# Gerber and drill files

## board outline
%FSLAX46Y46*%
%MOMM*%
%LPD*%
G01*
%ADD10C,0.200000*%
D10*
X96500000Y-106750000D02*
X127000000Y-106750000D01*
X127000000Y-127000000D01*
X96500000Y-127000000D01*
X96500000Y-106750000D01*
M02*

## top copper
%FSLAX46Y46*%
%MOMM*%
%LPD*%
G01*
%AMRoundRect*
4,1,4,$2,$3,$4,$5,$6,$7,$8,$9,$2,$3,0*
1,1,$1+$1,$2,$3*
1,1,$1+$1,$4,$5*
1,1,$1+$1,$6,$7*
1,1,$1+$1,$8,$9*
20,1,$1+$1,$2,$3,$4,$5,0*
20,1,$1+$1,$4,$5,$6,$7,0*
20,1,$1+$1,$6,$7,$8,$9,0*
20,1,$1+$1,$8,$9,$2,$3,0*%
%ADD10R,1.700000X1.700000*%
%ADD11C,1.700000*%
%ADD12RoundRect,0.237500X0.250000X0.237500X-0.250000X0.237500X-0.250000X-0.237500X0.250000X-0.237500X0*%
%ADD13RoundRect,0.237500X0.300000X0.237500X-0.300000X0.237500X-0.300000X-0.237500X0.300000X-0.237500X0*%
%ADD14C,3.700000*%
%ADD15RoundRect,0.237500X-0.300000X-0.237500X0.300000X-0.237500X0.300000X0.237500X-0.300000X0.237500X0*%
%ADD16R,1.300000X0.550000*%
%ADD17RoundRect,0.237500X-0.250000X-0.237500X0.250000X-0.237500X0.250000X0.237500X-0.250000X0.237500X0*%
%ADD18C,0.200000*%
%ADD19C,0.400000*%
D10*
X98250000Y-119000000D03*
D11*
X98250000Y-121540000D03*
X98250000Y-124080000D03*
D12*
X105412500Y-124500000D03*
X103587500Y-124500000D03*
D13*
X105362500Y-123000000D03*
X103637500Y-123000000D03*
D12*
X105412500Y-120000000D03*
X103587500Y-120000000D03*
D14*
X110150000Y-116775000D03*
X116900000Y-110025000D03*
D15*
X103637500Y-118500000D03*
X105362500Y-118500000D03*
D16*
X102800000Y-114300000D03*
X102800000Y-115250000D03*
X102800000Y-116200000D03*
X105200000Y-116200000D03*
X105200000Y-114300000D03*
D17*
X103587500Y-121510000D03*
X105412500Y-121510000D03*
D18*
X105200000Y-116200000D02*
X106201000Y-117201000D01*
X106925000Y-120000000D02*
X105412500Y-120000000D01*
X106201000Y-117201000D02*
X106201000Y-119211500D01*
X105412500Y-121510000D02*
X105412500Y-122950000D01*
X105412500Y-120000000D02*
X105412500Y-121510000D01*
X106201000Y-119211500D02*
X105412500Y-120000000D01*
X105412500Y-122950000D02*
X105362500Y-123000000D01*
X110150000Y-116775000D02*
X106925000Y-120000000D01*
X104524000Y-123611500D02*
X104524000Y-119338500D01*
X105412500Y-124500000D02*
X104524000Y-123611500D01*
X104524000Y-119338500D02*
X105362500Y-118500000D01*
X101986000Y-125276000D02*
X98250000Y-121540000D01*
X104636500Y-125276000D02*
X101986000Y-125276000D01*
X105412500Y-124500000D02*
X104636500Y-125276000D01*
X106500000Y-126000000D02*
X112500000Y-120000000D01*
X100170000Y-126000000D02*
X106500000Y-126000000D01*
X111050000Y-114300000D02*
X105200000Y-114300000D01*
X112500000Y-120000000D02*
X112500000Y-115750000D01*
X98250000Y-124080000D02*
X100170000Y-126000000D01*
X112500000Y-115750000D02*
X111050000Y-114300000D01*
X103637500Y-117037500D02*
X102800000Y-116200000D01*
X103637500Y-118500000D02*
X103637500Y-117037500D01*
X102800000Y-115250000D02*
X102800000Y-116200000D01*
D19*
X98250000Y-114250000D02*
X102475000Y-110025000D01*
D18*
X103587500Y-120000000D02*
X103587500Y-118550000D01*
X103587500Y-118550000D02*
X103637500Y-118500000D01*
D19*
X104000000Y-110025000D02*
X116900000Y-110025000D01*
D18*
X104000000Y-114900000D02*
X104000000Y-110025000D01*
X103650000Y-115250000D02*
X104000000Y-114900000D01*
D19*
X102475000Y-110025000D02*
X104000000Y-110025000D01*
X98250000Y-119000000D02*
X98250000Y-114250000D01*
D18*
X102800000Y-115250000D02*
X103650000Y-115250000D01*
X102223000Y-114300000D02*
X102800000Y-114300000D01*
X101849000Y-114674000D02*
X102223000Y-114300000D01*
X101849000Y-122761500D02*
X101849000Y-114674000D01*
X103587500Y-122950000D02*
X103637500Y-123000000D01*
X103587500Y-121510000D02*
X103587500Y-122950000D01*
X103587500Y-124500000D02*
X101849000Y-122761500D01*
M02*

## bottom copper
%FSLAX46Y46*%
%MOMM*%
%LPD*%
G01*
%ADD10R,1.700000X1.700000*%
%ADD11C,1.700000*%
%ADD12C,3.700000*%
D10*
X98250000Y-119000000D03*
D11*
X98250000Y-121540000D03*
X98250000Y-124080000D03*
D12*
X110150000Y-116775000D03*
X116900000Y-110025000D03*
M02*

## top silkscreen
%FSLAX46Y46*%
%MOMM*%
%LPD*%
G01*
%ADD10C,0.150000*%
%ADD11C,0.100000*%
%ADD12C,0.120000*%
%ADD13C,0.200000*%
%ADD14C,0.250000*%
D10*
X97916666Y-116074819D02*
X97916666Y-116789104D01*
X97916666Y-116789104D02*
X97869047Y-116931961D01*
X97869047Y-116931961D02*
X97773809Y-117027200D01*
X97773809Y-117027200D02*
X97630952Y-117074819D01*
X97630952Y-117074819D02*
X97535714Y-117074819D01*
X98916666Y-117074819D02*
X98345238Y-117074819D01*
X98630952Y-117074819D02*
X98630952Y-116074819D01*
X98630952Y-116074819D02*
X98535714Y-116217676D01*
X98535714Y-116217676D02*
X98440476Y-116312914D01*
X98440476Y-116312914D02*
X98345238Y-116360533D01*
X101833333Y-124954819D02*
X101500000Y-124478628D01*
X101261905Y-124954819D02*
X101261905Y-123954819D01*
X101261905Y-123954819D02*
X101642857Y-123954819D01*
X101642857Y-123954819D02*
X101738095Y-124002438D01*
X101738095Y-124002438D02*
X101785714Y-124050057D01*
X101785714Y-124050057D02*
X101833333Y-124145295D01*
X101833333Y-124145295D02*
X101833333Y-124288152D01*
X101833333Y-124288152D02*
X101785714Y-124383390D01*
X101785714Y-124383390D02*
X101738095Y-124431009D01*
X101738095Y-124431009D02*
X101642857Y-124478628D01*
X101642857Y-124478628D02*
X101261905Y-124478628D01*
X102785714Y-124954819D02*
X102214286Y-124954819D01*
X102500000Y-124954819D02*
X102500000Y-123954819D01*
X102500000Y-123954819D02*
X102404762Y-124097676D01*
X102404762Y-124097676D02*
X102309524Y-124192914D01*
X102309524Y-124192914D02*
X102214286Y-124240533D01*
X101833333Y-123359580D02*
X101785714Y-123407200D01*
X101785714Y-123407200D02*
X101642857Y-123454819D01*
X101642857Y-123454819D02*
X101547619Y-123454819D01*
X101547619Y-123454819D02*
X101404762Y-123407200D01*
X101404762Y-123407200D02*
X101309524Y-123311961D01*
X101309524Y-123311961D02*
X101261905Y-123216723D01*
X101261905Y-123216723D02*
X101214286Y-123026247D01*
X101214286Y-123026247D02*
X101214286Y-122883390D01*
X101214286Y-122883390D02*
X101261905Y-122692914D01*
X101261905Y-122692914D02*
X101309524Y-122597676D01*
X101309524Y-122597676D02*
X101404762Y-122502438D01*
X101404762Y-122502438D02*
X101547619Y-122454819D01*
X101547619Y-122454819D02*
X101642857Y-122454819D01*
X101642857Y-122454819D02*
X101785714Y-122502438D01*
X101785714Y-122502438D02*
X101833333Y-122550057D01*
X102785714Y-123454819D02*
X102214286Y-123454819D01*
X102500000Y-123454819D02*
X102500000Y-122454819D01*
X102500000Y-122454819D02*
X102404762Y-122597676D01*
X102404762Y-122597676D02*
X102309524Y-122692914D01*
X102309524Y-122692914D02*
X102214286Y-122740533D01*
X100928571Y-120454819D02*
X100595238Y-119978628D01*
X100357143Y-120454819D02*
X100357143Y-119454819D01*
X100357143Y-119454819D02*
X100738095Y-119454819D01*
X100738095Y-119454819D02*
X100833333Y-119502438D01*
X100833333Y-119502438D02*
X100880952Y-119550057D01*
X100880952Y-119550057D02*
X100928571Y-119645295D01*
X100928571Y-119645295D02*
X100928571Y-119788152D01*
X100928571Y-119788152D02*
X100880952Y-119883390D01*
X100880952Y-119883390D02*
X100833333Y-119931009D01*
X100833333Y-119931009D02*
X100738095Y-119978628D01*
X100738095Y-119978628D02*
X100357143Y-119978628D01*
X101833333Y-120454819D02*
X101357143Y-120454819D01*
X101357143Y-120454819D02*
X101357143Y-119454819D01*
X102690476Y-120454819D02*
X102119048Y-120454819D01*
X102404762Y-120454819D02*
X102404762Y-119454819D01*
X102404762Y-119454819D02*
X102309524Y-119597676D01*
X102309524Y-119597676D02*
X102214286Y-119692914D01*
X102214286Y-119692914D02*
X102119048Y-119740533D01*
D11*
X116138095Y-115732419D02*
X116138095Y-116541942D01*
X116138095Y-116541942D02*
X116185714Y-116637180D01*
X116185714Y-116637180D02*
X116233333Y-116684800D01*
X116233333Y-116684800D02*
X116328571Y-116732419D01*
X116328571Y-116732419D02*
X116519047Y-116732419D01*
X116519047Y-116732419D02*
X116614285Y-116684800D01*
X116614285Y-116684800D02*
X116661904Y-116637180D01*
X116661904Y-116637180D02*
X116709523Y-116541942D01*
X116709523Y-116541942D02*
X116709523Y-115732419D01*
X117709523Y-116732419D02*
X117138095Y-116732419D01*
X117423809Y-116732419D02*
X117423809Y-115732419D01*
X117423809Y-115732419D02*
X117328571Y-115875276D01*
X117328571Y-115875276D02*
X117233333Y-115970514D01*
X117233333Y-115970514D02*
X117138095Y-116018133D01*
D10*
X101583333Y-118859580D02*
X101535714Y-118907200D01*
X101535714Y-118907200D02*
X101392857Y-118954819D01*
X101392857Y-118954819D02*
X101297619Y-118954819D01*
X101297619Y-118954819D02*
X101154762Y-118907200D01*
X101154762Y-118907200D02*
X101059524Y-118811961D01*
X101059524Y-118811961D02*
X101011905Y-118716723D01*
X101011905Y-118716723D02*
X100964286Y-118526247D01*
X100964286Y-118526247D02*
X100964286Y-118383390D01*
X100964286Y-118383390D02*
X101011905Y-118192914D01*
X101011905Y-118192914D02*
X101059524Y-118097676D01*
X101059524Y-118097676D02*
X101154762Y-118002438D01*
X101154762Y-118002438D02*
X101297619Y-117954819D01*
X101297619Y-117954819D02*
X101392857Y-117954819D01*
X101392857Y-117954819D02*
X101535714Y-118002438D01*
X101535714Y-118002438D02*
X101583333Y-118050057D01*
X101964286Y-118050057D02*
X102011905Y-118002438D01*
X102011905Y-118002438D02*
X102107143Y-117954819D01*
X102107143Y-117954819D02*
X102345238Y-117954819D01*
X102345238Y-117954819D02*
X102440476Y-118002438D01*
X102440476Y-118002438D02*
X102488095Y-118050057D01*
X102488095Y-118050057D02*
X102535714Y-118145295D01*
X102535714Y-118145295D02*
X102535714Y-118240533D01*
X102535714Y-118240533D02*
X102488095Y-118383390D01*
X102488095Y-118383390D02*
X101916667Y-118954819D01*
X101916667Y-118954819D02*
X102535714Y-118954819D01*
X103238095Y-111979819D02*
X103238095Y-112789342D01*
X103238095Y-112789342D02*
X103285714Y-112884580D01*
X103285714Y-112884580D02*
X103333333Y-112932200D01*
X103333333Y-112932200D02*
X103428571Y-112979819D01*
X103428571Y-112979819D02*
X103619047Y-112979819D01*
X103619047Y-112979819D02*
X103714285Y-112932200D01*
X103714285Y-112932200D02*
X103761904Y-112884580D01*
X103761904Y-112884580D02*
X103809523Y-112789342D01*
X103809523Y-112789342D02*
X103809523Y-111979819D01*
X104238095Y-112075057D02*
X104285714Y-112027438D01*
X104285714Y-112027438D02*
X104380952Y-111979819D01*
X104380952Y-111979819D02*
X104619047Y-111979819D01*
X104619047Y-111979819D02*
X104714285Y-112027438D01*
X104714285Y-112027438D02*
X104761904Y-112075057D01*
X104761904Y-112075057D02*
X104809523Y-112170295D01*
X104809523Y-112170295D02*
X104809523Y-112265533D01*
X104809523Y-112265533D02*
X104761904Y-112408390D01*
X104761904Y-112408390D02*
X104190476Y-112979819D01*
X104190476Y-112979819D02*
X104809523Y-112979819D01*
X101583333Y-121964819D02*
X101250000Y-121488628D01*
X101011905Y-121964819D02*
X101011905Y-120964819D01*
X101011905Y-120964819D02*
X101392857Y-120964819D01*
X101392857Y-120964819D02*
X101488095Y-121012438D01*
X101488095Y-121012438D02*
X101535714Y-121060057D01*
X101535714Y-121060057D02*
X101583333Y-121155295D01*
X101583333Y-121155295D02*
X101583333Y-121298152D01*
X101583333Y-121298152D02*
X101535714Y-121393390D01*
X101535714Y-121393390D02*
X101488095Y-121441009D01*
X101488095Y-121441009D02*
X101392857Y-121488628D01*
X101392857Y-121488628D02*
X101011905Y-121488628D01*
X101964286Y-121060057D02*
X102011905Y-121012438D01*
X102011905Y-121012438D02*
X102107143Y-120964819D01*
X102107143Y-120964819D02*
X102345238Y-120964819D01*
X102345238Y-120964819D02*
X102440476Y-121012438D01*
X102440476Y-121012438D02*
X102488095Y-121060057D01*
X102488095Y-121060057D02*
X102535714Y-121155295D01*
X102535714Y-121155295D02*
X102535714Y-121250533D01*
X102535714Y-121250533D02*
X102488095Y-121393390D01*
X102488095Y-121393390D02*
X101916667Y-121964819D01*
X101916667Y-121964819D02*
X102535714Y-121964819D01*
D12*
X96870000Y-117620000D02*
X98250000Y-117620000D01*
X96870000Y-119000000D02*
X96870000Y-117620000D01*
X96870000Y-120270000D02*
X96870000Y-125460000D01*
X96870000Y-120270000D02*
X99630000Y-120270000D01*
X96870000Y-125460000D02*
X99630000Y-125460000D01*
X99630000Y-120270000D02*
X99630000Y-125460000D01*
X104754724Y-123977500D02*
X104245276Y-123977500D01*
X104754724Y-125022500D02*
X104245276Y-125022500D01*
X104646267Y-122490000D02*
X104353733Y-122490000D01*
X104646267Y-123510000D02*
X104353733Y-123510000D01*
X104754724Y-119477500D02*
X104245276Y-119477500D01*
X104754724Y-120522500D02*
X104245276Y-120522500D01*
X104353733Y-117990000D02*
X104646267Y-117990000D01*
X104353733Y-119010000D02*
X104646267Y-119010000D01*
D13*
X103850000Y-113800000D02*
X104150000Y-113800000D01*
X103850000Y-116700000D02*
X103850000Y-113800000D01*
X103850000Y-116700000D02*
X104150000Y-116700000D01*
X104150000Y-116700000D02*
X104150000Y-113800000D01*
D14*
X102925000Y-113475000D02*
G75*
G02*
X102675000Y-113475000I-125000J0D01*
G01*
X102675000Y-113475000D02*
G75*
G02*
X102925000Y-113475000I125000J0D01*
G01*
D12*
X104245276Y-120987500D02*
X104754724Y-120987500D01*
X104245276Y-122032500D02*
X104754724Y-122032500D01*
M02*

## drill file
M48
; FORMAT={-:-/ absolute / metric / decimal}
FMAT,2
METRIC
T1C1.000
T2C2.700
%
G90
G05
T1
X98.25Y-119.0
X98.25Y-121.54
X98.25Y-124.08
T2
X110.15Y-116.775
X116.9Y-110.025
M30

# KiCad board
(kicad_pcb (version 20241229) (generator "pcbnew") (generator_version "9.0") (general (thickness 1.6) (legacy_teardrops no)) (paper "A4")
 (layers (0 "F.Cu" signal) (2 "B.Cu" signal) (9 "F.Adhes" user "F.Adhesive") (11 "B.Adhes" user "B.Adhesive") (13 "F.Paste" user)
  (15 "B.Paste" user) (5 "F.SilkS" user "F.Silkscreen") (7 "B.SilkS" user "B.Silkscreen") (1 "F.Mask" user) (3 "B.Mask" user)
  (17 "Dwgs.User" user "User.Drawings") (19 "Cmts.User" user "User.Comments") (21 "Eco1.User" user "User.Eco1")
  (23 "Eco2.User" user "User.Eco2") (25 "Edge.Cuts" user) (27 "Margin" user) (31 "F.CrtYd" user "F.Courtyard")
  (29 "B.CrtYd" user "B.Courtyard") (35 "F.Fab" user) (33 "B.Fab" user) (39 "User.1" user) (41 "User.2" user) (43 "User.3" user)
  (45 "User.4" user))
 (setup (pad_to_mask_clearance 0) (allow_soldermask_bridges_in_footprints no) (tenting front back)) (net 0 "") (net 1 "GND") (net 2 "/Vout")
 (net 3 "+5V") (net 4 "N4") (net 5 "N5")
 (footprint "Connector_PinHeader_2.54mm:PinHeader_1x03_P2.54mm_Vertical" (layer "F.Cu") (at 98.25 119)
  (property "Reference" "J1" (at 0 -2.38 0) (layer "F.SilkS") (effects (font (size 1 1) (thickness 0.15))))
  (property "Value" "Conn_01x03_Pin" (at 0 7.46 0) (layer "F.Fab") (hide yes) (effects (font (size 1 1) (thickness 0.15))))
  (fp_line (start -1.38 -1.38) (end 0 -1.38) (stroke (width 0.12) (type solid)) (layer "F.SilkS"))
  (fp_line (start -1.38 0) (end -1.38 -1.38) (stroke (width 0.12) (type solid)) (layer "F.SilkS"))
  (fp_line (start -1.38 1.27) (end -1.38 6.46) (stroke (width 0.12) (type solid)) (layer "F.SilkS"))
  (fp_line (start -1.38 1.27) (end 1.38 1.27) (stroke (width 0.12) (type solid)) (layer "F.SilkS"))
  (fp_line (start -1.38 6.46) (end 1.38 6.46) (stroke (width 0.12) (type solid)) (layer "F.SilkS"))
  (fp_line (start 1.38 1.27) (end 1.38 6.46) (stroke (width 0.12) (type solid)) (layer "F.SilkS"))
  (pad "1" thru_hole rect (at 0 0) (size 1.7 1.7) (drill 1) (layers "*.Cu" "*.Mask") (remove_unused_layers no) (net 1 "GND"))
  (pad "2" thru_hole circle (at 0 2.54) (size 1.7 1.7) (drill 1) (layers "*.Cu" "*.Mask") (remove_unused_layers no) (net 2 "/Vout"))
  (pad "3" thru_hole circle (at 0 5.08) (size 1.7 1.7) (drill 1) (layers "*.Cu" "*.Mask") (remove_unused_layers no) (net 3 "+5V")))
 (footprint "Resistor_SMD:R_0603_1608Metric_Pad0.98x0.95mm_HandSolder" (layer "F.Cu") (at 104.5 124.5 180)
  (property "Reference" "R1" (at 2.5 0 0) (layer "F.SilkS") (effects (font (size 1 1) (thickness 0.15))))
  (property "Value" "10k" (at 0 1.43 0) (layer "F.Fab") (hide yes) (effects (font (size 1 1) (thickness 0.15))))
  (fp_line (start -0.254724 0.5225) (end 0.254724 0.5225) (stroke (width 0.12) (type solid)) (layer "F.SilkS"))
  (fp_line (start -0.254724 -0.5225) (end 0.254724 -0.5225) (stroke (width 0.12) (type solid)) (layer "F.SilkS"))
  (pad "1" smd roundrect (at -0.9125 0 180) (size 0.975 0.95) (layers "F.Cu" "F.Mask" "F.Paste") (roundrect_rratio 0.25) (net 2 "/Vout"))
  (pad "2" smd roundrect (at 0.9125 0 180) (size 0.975 0.95) (layers "F.Cu" "F.Mask" "F.Paste") (roundrect_rratio 0.25) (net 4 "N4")))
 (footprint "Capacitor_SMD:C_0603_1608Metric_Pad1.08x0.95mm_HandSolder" (layer "F.Cu") (at 104.5 123 180)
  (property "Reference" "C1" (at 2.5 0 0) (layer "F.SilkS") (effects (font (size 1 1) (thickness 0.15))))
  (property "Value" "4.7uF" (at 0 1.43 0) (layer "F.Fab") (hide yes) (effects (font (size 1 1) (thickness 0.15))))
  (fp_line (start -0.146267 0.51) (end 0.146267 0.51) (stroke (width 0.12) (type solid)) (layer "F.SilkS"))
  (fp_line (start -0.146267 -0.51) (end 0.146267 -0.51) (stroke (width 0.12) (type solid)) (layer "F.SilkS"))
  (pad "1" smd roundrect (at -0.8625 0 180) (size 1.075 0.95) (layers "F.Cu" "F.Mask" "F.Paste") (roundrect_rratio 0.25) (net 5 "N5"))
  (pad "2" smd roundrect (at 0.8625 0 180) (size 1.075 0.95) (layers "F.Cu" "F.Mask" "F.Paste") (roundrect_rratio 0.25) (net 4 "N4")))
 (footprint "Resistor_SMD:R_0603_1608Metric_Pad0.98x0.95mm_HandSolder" (layer "F.Cu") (at 104.5 120 180)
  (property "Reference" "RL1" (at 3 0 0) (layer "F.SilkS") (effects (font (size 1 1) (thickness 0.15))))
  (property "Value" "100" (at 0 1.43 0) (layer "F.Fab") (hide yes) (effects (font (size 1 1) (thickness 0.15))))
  (fp_line (start -0.254724 0.5225) (end 0.254724 0.5225) (stroke (width 0.12) (type solid)) (layer "F.SilkS"))
  (fp_line (start -0.254724 -0.5225) (end 0.254724 -0.5225) (stroke (width 0.12) (type solid)) (layer "F.SilkS"))
  (pad "1" smd roundrect (at -0.9125 0 180) (size 0.975 0.95) (layers "F.Cu" "F.Mask" "F.Paste") (roundrect_rratio 0.25) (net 5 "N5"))
  (pad "2" smd roundrect (at 0.9125 0 180) (size 0.975 0.95) (layers "F.Cu" "F.Mask" "F.Paste") (roundrect_rratio 0.25) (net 1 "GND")))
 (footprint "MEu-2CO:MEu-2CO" (layer "F.Cu") (at 116.9 116.775)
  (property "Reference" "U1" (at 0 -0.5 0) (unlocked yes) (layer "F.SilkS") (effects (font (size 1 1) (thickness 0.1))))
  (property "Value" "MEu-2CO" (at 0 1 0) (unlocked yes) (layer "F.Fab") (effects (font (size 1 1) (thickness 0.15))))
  (pad "1" thru_hole circle (at -6.75 0) (size 3.7 3.7) (drill 2.7) (layers "*.Cu" "*.Mask") (remove_unused_layers no) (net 5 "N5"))
  (pad "2" thru_hole circle (at 0 -6.75) (size 3.7 3.7) (drill 2.7) (layers "*.Cu" "*.Mask") (remove_unused_layers no) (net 1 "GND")))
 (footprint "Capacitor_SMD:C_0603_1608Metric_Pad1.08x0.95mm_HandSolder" (layer "F.Cu") (at 104.5 118.5)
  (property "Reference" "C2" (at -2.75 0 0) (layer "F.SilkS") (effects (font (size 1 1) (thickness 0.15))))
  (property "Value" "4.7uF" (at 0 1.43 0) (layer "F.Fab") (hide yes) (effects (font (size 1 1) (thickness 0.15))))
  (fp_line (start -0.146267 -0.51) (end 0.146267 -0.51) (stroke (width 0.12) (type solid)) (layer "F.SilkS"))
  (fp_line (start -0.146267 0.51) (end 0.146267 0.51) (stroke (width 0.12) (type solid)) (layer "F.SilkS"))
  (pad "1" smd roundrect (at -0.8625 0) (size 1.075 0.95) (layers "F.Cu" "F.Mask" "F.Paste") (roundrect_rratio 0.25) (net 1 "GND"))
  (pad "2" smd roundrect (at 0.8625 0) (size 1.075 0.95) (layers "F.Cu" "F.Mask" "F.Paste") (roundrect_rratio 0.25) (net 2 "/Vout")))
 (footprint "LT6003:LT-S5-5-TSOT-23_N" (layer "F.Cu") (at 104 115.25)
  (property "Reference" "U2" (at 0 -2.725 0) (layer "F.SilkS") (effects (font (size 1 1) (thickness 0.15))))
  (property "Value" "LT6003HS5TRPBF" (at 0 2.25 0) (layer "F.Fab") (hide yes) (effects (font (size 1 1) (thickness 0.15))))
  (fp_line (start -0.15 -1.45) (end 0.15 -1.45) (stroke (width 0.2) (type solid)) (layer "F.SilkS"))
  (fp_line (start -0.15 1.45) (end -0.15 -1.45) (stroke (width 0.2) (type solid)) (layer "F.SilkS"))
  (fp_line (start -0.15 1.45) (end 0.15 1.45) (stroke (width 0.2) (type solid)) (layer "F.SilkS"))
  (fp_line (start 0.15 1.45) (end 0.15 -1.45) (stroke (width 0.2) (type solid)) (layer "F.SilkS"))
  (fp_circle (center -1.2 -1.775) (end -1.2 -1.9) (stroke (width 0.25) (type solid)) (fill no) (layer "F.SilkS"))
  (pad "1" smd rect (at -1.2 -0.95 90) (size 0.55 1.3) (layers "F.Cu" "F.Mask" "F.Paste") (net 4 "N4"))
  (pad "2" smd rect (at -1.2 0 90) (size 0.55 1.3) (layers "F.Cu" "F.Mask" "F.Paste") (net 1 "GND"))
  (pad "3" smd rect (at -1.2 0.95 90) (size 0.55 1.3) (layers "F.Cu" "F.Mask" "F.Paste") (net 1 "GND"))
  (pad "4" smd rect (at 1.2 0.95 90) (size 0.55 1.3) (layers "F.Cu" "F.Mask" "F.Paste") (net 5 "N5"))
  (pad "5" smd rect (at 1.2 -0.95 90) (size 0.55 1.3) (layers "F.Cu" "F.Mask" "F.Paste") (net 3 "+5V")))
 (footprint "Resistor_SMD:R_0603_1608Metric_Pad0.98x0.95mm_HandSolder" (layer "F.Cu") (at 104.5 121.51)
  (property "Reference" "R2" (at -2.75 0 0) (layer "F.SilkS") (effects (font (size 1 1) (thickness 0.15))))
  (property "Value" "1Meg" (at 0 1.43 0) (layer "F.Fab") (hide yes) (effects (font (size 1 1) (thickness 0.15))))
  (fp_line (start -0.254724 -0.5225) (end 0.254724 -0.5225) (stroke (width 0.12) (type solid)) (layer "F.SilkS"))
  (fp_line (start -0.254724 0.5225) (end 0.254724 0.5225) (stroke (width 0.12) (type solid)) (layer "F.SilkS"))
  (pad "1" smd roundrect (at -0.9125 0) (size 0.975 0.95) (layers "F.Cu" "F.Mask" "F.Paste") (roundrect_rratio 0.25) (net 4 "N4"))
  (pad "2" smd roundrect (at 0.9125 0) (size 0.975 0.95) (layers "F.Cu" "F.Mask" "F.Paste") (roundrect_rratio 0.25) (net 5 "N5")))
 (gr_rect (start 96.5 106.75) (end 127 127) (stroke (width 0.2) (type solid)) (fill no) (layer "Edge.Cuts"))
 (segment (start 105.2 116.2) (end 106.201 117.201) (width 0.2) (layer "F.Cu") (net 5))
 (segment (start 106.925 120) (end 105.4125 120) (width 0.2) (layer "F.Cu") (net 5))
 (segment (start 106.201 117.201) (end 106.201 119.2115) (width 0.2) (layer "F.Cu") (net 5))
 (segment (start 105.4125 121.51) (end 105.4125 122.95) (width 0.2) (layer "F.Cu") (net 5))
 (segment (start 105.4125 120) (end 105.4125 121.51) (width 0.2) (layer "F.Cu") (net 5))
 (segment (start 106.201 119.2115) (end 105.4125 120) (width 0.2) (layer "F.Cu") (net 5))
 (segment (start 105.4125 122.95) (end 105.3625 123) (width 0.2) (layer "F.Cu") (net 5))
 (segment (start 110.15 116.775) (end 106.925 120) (width 0.2) (layer "F.Cu") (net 5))
 (segment (start 104.524 123.6115) (end 104.524 119.3385) (width 0.2) (layer "F.Cu") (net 2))
 (segment (start 105.4125 124.5) (end 104.524 123.6115) (width 0.2) (layer "F.Cu") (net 2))
 (segment (start 104.524 119.3385) (end 105.3625 118.5) (width 0.2) (layer "F.Cu") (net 2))
 (segment (start 101.986 125.276) (end 98.25 121.54) (width 0.2) (layer "F.Cu") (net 2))
 (segment (start 104.6365 125.276) (end 101.986 125.276) (width 0.2) (layer "F.Cu") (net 2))
 (segment (start 105.4125 124.5) (end 104.6365 125.276) (width 0.2) (layer "F.Cu") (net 2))
 (segment (start 106.5 126) (end 112.5 120) (width 0.2) (layer "F.Cu") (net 3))
 (segment (start 100.17 126) (end 106.5 126) (width 0.2) (layer "F.Cu") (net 3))
 (segment (start 111.05 114.3) (end 105.2 114.3) (width 0.2) (layer "F.Cu") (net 3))
 (segment (start 112.5 120) (end 112.5 115.75) (width 0.2) (layer "F.Cu") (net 3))
 (segment (start 98.25 124.08) (end 100.17 126) (width 0.2) (layer "F.Cu") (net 3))
 (segment (start 112.5 115.75) (end 111.05 114.3) (width 0.2) (layer "F.Cu") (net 3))
 (segment (start 103.6375 117.0375) (end 102.8 116.2) (width 0.2) (layer "F.Cu") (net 1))
 (segment (start 103.6375 118.5) (end 103.6375 117.0375) (width 0.2) (layer "F.Cu") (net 1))
 (segment (start 102.8 115.25) (end 102.8 116.2) (width 0.2) (layer "F.Cu") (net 1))
 (segment (start 98.25 114.25) (end 102.475 110.025) (width 0.4) (layer "F.Cu") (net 1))
 (segment (start 103.5875 120) (end 103.5875 118.55) (width 0.2) (layer "F.Cu") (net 1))
 (segment (start 103.5875 118.55) (end 103.6375 118.5) (width 0.2) (layer "F.Cu") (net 1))
 (segment (start 104 110.025) (end 116.9 110.025) (width 0.4) (layer "F.Cu") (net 1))
 (segment (start 104 114.9) (end 104 110.025) (width 0.2) (layer "F.Cu") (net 1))
 (segment (start 103.65 115.25) (end 104 114.9) (width 0.2) (layer "F.Cu") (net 1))
 (segment (start 102.475 110.025) (end 104 110.025) (width 0.4) (layer "F.Cu") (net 1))
 (segment (start 98.25 119) (end 98.25 114.25) (width 0.4) (layer "F.Cu") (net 1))
 (segment (start 102.8 115.25) (end 103.65 115.25) (width 0.2) (layer "F.Cu") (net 1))
 (segment (start 102.223 114.3) (end 102.8 114.3) (width 0.2) (layer "F.Cu") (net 4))
 (segment (start 101.849 114.674) (end 102.223 114.3) (width 0.2) (layer "F.Cu") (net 4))
 (segment (start 101.849 122.7615) (end 101.849 114.674) (width 0.2) (layer "F.Cu") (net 4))
 (segment (start 103.5875 122.95) (end 103.6375 123) (width 0.2) (layer "F.Cu") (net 4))
 (segment (start 103.5875 121.51) (end 103.5875 122.95) (width 0.2) (layer "F.Cu") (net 4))
 (segment (start 103.5875 124.5) (end 101.849 122.7615) (width 0.2) (layer "F.Cu") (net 4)))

